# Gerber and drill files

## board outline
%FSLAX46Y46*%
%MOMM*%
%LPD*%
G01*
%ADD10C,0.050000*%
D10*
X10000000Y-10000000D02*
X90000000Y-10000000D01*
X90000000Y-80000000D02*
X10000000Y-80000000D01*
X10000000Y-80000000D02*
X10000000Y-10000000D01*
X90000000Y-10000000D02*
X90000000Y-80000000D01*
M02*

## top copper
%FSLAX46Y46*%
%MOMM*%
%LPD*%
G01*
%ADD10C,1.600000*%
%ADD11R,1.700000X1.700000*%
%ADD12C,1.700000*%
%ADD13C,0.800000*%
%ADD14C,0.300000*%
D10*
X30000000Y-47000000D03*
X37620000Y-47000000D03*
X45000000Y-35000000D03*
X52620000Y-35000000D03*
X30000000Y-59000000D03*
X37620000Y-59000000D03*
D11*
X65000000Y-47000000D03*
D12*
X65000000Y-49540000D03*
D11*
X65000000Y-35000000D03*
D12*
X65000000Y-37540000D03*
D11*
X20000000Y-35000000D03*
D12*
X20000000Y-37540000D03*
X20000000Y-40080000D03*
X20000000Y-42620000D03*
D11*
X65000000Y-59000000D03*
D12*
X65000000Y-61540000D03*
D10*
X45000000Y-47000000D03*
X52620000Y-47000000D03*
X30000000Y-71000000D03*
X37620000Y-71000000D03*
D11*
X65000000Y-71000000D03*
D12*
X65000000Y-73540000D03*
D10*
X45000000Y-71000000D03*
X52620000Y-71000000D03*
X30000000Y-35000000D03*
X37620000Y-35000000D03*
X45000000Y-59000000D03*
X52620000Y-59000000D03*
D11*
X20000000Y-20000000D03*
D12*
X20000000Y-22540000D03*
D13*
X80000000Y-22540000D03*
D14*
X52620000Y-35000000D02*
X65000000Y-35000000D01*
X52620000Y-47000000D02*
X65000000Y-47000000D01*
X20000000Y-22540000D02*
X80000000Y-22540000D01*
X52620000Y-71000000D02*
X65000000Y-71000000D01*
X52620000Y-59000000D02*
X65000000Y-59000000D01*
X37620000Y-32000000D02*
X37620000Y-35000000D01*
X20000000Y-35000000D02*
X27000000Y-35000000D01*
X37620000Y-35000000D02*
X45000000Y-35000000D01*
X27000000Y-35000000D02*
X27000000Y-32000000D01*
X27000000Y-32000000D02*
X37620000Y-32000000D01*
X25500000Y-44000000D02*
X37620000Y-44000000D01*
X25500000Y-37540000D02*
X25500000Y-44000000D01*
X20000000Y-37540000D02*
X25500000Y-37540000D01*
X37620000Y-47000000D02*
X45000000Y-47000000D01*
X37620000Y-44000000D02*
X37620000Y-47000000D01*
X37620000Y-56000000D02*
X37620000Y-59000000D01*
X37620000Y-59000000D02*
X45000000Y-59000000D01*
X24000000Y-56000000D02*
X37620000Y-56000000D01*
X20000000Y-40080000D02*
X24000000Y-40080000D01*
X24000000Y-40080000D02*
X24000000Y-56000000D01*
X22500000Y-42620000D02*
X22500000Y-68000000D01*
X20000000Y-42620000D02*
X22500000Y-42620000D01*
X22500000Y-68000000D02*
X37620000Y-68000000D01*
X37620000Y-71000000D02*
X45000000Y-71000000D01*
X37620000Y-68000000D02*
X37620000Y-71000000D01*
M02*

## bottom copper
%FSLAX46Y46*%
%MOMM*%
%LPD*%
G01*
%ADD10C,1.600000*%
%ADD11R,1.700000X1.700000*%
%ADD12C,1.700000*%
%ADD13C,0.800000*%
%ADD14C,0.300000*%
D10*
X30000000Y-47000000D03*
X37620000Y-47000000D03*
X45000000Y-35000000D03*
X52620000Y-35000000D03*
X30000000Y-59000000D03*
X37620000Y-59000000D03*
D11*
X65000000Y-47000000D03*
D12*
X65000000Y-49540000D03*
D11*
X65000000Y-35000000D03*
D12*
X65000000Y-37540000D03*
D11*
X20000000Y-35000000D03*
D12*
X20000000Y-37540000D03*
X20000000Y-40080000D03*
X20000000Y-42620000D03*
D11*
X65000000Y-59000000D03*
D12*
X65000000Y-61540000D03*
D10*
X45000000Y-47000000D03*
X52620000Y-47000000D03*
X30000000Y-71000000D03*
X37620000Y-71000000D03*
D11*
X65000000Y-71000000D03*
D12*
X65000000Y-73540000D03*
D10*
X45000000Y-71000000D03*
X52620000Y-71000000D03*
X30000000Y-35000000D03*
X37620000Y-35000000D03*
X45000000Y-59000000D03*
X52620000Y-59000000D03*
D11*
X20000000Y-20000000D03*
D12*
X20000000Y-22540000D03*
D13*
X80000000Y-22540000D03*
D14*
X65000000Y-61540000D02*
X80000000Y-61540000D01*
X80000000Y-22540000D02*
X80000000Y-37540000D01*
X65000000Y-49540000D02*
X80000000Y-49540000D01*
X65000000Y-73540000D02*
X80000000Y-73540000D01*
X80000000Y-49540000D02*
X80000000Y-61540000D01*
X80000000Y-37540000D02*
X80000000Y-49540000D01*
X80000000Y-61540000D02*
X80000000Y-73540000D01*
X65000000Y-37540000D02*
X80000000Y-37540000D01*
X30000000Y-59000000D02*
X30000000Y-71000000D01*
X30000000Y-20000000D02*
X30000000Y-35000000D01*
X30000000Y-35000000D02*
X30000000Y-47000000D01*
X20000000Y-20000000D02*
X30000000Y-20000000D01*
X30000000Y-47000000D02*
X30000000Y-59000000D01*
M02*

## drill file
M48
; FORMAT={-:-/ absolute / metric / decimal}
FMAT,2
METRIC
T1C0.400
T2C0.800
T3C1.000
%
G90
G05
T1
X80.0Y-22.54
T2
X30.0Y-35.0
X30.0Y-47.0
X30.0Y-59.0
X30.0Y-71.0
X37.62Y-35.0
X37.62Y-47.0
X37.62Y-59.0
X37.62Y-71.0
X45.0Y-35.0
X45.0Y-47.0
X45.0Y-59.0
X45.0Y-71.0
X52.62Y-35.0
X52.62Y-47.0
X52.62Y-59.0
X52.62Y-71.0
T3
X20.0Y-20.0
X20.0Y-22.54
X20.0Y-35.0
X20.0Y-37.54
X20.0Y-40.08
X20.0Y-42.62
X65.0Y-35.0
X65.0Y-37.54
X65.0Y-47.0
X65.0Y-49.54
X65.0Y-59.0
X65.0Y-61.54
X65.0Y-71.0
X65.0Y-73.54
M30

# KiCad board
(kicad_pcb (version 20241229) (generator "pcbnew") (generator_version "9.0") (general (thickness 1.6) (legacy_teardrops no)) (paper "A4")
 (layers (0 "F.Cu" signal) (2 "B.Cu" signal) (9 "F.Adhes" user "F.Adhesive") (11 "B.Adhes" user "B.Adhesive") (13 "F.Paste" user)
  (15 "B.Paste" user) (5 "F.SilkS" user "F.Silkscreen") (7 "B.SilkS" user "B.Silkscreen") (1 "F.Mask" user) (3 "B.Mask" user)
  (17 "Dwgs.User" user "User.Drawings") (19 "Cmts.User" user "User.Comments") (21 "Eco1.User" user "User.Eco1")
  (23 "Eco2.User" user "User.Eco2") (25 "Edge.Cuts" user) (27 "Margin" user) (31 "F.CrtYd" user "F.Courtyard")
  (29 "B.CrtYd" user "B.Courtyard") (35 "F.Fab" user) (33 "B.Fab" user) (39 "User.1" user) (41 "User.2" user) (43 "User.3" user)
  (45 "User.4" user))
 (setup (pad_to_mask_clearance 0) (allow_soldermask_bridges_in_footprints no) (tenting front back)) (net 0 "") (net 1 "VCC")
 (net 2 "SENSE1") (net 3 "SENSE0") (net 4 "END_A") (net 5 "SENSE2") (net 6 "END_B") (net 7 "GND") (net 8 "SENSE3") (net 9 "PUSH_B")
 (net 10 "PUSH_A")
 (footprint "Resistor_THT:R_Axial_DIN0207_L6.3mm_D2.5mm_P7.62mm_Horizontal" (layer "F.Cu") (at 30 47)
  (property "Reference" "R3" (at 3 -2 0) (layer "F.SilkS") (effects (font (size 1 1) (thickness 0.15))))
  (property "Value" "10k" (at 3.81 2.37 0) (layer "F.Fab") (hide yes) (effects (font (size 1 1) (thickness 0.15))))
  (pad "1" thru_hole circle (at 0 0) (size 1.6 1.6) (drill 0.8) (layers "*.Cu" "*.Mask") (remove_unused_layers no) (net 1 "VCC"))
  (pad "2" thru_hole circle (at 7.62 0) (size 1.6 1.6) (drill 0.8) (layers "*.Cu" "*.Mask") (remove_unused_layers no) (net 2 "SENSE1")))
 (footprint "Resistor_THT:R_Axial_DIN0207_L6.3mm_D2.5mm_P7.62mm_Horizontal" (layer "F.Cu") (at 45 35)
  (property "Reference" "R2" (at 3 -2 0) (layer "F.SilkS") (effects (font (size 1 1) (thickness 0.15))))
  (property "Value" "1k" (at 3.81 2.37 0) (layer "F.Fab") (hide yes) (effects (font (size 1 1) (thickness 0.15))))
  (pad "1" thru_hole circle (at 0 0) (size 1.6 1.6) (drill 0.8) (layers "*.Cu" "*.Mask") (remove_unused_layers no) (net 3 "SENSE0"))
  (pad "2" thru_hole circle (at 7.62 0) (size 1.6 1.6) (drill 0.8) (layers "*.Cu" "*.Mask") (remove_unused_layers no) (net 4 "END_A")))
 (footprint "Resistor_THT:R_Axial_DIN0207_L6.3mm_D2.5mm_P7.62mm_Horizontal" (layer "F.Cu") (at 30 59)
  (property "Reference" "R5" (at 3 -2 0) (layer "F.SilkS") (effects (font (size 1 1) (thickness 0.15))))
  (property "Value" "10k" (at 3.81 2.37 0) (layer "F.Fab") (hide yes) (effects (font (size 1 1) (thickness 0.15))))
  (pad "1" thru_hole circle (at 0 0) (size 1.6 1.6) (drill 0.8) (layers "*.Cu" "*.Mask") (remove_unused_layers no) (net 1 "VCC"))
  (pad "2" thru_hole circle (at 7.62 0) (size 1.6 1.6) (drill 0.8) (layers "*.Cu" "*.Mask") (remove_unused_layers no) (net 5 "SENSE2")))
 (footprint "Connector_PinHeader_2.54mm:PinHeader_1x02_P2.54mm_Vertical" (layer "F.Cu") (at 65 47)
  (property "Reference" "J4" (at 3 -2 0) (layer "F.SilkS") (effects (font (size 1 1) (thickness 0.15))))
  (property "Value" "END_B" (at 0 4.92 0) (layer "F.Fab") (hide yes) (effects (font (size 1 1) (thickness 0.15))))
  (pad "1" thru_hole rect (at 0 0) (size 1.7 1.7) (drill 1) (layers "*.Cu" "*.Mask") (remove_unused_layers no) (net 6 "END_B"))
  (pad "2" thru_hole circle (at 0 2.54) (size 1.7 1.7) (drill 1) (layers "*.Cu" "*.Mask") (remove_unused_layers no) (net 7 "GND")))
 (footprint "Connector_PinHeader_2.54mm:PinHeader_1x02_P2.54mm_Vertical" (layer "F.Cu") (at 65 35)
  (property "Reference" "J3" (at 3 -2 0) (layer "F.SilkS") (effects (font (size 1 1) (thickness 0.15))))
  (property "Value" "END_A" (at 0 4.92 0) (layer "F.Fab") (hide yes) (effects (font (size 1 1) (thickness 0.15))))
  (pad "1" thru_hole rect (at 0 0) (size 1.7 1.7) (drill 1) (layers "*.Cu" "*.Mask") (remove_unused_layers no) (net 4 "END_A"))
  (pad "2" thru_hole circle (at 0 2.54) (size 1.7 1.7) (drill 1) (layers "*.Cu" "*.Mask") (remove_unused_layers no) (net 7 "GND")))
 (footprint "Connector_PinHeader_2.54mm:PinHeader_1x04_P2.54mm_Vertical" (layer "F.Cu") (at 20 35)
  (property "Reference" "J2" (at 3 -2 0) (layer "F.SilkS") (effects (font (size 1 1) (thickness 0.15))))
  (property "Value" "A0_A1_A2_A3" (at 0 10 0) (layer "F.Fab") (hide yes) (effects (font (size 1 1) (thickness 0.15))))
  (pad "1" thru_hole rect (at 0 0) (size 1.7 1.7) (drill 1) (layers "*.Cu" "*.Mask") (remove_unused_layers no) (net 3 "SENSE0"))
  (pad "2" thru_hole circle (at 0 2.54) (size 1.7 1.7) (drill 1) (layers "*.Cu" "*.Mask") (remove_unused_layers no) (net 2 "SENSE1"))
  (pad "3" thru_hole circle (at 0 5.08) (size 1.7 1.7) (drill 1) (layers "*.Cu" "*.Mask") (remove_unused_layers no) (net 5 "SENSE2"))
  (pad "4" thru_hole circle (at 0 7.62) (size 1.7 1.7) (drill 1) (layers "*.Cu" "*.Mask") (remove_unused_layers no) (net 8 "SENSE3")))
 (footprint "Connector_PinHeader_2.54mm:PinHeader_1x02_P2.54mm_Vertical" (layer "F.Cu") (at 65 59)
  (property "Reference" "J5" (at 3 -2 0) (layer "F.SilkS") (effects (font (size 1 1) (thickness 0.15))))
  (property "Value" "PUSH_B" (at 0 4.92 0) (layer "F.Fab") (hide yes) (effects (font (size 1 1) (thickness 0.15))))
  (pad "1" thru_hole rect (at 0 0) (size 1.7 1.7) (drill 1) (layers "*.Cu" "*.Mask") (remove_unused_layers no) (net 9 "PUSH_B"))
  (pad "2" thru_hole circle (at 0 2.54) (size 1.7 1.7) (drill 1) (layers "*.Cu" "*.Mask") (remove_unused_layers no) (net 7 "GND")))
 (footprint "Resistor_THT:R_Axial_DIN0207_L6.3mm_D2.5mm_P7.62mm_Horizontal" (layer "F.Cu") (at 45 47)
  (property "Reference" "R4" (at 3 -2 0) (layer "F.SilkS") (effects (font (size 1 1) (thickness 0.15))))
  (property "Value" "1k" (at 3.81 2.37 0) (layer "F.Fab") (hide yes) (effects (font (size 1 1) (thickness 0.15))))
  (pad "1" thru_hole circle (at 0 0) (size 1.6 1.6) (drill 0.8) (layers "*.Cu" "*.Mask") (remove_unused_layers no) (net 2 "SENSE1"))
  (pad "2" thru_hole circle (at 7.62 0) (size 1.6 1.6) (drill 0.8) (layers "*.Cu" "*.Mask") (remove_unused_layers no) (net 6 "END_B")))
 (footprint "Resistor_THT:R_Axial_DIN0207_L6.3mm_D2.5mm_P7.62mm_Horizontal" (layer "F.Cu") (at 30 71)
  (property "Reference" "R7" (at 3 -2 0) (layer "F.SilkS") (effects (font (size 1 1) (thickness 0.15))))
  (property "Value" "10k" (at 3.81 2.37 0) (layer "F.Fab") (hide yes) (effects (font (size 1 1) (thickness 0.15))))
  (pad "1" thru_hole circle (at 0 0) (size 1.6 1.6) (drill 0.8) (layers "*.Cu" "*.Mask") (remove_unused_layers no) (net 1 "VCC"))
  (pad "2" thru_hole circle (at 7.62 0) (size 1.6 1.6) (drill 0.8) (layers "*.Cu" "*.Mask") (remove_unused_layers no) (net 8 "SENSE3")))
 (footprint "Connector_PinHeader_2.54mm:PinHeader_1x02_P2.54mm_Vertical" (layer "F.Cu") (at 65 71)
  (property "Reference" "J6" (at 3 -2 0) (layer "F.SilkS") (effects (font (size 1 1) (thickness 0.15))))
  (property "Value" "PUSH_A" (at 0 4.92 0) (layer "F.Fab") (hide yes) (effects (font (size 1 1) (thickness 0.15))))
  (pad "1" thru_hole rect (at 0 0) (size 1.7 1.7) (drill 1) (layers "*.Cu" "*.Mask") (remove_unused_layers no) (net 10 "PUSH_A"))
  (pad "2" thru_hole circle (at 0 2.54) (size 1.7 1.7) (drill 1) (layers "*.Cu" "*.Mask") (remove_unused_layers no) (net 7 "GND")))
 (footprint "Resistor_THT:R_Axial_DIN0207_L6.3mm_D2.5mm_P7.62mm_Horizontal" (layer "F.Cu") (at 45 71)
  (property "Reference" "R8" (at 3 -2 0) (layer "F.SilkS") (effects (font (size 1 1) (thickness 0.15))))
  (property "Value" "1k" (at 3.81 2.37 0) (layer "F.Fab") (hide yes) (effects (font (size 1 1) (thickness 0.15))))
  (pad "1" thru_hole circle (at 0 0) (size 1.6 1.6) (drill 0.8) (layers "*.Cu" "*.Mask") (remove_unused_layers no) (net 8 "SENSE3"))
  (pad "2" thru_hole circle (at 7.62 0) (size 1.6 1.6) (drill 0.8) (layers "*.Cu" "*.Mask") (remove_unused_layers no) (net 10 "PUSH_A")))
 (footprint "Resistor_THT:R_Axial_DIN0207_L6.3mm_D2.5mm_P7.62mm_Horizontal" (layer "F.Cu") (at 30 35)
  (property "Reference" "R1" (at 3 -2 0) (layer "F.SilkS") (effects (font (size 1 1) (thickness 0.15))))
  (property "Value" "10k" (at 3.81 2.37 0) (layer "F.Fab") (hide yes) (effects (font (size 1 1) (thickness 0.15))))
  (pad "1" thru_hole circle (at 0 0) (size 1.6 1.6) (drill 0.8) (layers "*.Cu" "*.Mask") (remove_unused_layers no) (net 1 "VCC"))
  (pad "2" thru_hole circle (at 7.62 0) (size 1.6 1.6) (drill 0.8) (layers "*.Cu" "*.Mask") (remove_unused_layers no) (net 3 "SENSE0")))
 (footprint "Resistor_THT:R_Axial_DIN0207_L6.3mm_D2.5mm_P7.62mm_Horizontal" (layer "F.Cu") (at 45 59)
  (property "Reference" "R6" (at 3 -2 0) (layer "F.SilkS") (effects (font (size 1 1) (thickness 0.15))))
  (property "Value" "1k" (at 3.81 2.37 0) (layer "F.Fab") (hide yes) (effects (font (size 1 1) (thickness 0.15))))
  (pad "1" thru_hole circle (at 0 0) (size 1.6 1.6) (drill 0.8) (layers "*.Cu" "*.Mask") (remove_unused_layers no) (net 5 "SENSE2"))
  (pad "2" thru_hole circle (at 7.62 0) (size 1.6 1.6) (drill 0.8) (layers "*.Cu" "*.Mask") (remove_unused_layers no) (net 9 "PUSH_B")))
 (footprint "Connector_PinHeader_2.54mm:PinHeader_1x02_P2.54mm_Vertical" (layer "F.Cu") (at 20 20)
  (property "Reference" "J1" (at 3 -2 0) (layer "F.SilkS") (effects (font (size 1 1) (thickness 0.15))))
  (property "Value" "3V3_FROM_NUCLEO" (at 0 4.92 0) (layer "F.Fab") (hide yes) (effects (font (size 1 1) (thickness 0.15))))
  (pad "1" thru_hole rect (at 0 0) (size 1.7 1.7) (drill 1) (layers "*.Cu" "*.Mask") (remove_unused_layers no) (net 1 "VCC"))
  (pad "2" thru_hole circle (at 0 2.54) (size 1.7 1.7) (drill 1) (layers "*.Cu" "*.Mask") (remove_unused_layers no) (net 7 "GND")))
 (gr_line (start 10 10) (end 90 10) (stroke (width 0.05) (type default)) (layer "Edge.Cuts"))
 (gr_line (start 90 80) (end 10 80) (stroke (width 0.05) (type default)) (layer "Edge.Cuts"))
 (gr_line (start 10 80) (end 10 10) (stroke (width 0.05) (type default)) (layer "Edge.Cuts"))
 (gr_line (start 90 10) (end 90 80) (stroke (width 0.05) (type default)) (layer "Edge.Cuts"))
 (segment (start 52.62 35) (end 65 35) (width 0.3) (layer "F.Cu") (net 4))
 (segment (start 52.62 47) (end 65 47) (width 0.3) (layer "F.Cu") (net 6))
 (segment (start 20 22.54) (end 80 22.54) (width 0.3) (layer "F.Cu") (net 7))
 (via (at 80 22.54) (size 0.8) (drill 0.4) (layers "F.Cu" "B.Cu") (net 7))
 (segment (start 65 61.54) (end 80 61.54) (width 0.3) (layer "B.Cu") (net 7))
 (segment (start 80 22.54) (end 80 37.54) (width 0.3) (layer "B.Cu") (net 7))
 (segment (start 65 49.54) (end 80 49.54) (width 0.3) (layer "B.Cu") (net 7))
 (segment (start 65 73.54) (end 80 73.54) (width 0.3) (layer "B.Cu") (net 7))
 (segment (start 80 49.54) (end 80 61.54) (width 0.3) (layer "B.Cu") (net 7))
 (segment (start 80 37.54) (end 80 49.54) (width 0.3) (layer "B.Cu") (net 7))
 (segment (start 80 61.54) (end 80 73.54) (width 0.3) (layer "B.Cu") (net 7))
 (segment (start 65 37.54) (end 80 37.54) (width 0.3) (layer "B.Cu") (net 7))
 (segment (start 52.62 71) (end 65 71) (width 0.3) (layer "F.Cu") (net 10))
 (segment (start 52.62 59) (end 65 59) (width 0.3) (layer "F.Cu") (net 9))
 (segment (start 37.62 32) (end 37.62 35) (width 0.3) (layer "F.Cu") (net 3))
 (segment (start 20 35) (end 27 35) (width 0.3) (layer "F.Cu") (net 3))
 (segment (start 37.62 35) (end 45 35) (width 0.3) (layer "F.Cu") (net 3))
 (segment (start 27 35) (end 27 32) (width 0.3) (layer "F.Cu") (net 3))
 (segment (start 27 32) (end 37.62 32) (width 0.3) (layer "F.Cu") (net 3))
 (segment (start 25.5 44) (end 37.62 44) (width 0.3) (layer "F.Cu") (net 2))
 (segment (start 25.5 37.54) (end 25.5 44) (width 0.3) (layer "F.Cu") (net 2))
 (segment (start 20 37.54) (end 25.5 37.54) (width 0.3) (layer "F.Cu") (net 2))
 (segment (start 37.62 47) (end 45 47) (width 0.3) (layer "F.Cu") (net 2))
 (segment (start 37.62 44) (end 37.62 47) (width 0.3) (layer "F.Cu") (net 2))
 (segment (start 37.62 56) (end 37.62 59) (width 0.3) (layer "F.Cu") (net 5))
 (segment (start 37.62 59) (end 45 59) (width 0.3) (layer "F.Cu") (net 5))
 (segment (start 24 56) (end 37.62 56) (width 0.3) (layer "F.Cu") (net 5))
 (segment (start 20 40.08) (end 24 40.08) (width 0.3) (layer "F.Cu") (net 5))
 (segment (start 24 40.08) (end 24 56) (width 0.3) (layer "F.Cu") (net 5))
 (segment (start 22.5 42.62) (end 22.5 68) (width 0.3) (layer "F.Cu") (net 8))
 (segment (start 20 42.62) (end 22.5 42.62) (width 0.3) (layer "F.Cu") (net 8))
 (segment (start 22.5 68) (end 37.62 68) (width 0.3) (layer "F.Cu") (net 8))
 (segment (start 37.62 71) (end 45 71) (width 0.3) (layer "F.Cu") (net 8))
 (segment (start 37.62 68) (end 37.62 71) (width 0.3) (layer "F.Cu") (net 8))
 (segment (start 30 59) (end 30 71) (width 0.3) (layer "B.Cu") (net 1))
 (segment (start 30 20) (end 30 35) (width 0.3) (layer "B.Cu") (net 1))
 (segment (start 30 35) (end 30 47) (width 0.3) (layer "B.Cu") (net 1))
 (segment (start 20 20) (end 30 20) (width 0.3) (layer "B.Cu") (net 1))
 (segment (start 30 47) (end 30 59) (width 0.3) (layer "B.Cu") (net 1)))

